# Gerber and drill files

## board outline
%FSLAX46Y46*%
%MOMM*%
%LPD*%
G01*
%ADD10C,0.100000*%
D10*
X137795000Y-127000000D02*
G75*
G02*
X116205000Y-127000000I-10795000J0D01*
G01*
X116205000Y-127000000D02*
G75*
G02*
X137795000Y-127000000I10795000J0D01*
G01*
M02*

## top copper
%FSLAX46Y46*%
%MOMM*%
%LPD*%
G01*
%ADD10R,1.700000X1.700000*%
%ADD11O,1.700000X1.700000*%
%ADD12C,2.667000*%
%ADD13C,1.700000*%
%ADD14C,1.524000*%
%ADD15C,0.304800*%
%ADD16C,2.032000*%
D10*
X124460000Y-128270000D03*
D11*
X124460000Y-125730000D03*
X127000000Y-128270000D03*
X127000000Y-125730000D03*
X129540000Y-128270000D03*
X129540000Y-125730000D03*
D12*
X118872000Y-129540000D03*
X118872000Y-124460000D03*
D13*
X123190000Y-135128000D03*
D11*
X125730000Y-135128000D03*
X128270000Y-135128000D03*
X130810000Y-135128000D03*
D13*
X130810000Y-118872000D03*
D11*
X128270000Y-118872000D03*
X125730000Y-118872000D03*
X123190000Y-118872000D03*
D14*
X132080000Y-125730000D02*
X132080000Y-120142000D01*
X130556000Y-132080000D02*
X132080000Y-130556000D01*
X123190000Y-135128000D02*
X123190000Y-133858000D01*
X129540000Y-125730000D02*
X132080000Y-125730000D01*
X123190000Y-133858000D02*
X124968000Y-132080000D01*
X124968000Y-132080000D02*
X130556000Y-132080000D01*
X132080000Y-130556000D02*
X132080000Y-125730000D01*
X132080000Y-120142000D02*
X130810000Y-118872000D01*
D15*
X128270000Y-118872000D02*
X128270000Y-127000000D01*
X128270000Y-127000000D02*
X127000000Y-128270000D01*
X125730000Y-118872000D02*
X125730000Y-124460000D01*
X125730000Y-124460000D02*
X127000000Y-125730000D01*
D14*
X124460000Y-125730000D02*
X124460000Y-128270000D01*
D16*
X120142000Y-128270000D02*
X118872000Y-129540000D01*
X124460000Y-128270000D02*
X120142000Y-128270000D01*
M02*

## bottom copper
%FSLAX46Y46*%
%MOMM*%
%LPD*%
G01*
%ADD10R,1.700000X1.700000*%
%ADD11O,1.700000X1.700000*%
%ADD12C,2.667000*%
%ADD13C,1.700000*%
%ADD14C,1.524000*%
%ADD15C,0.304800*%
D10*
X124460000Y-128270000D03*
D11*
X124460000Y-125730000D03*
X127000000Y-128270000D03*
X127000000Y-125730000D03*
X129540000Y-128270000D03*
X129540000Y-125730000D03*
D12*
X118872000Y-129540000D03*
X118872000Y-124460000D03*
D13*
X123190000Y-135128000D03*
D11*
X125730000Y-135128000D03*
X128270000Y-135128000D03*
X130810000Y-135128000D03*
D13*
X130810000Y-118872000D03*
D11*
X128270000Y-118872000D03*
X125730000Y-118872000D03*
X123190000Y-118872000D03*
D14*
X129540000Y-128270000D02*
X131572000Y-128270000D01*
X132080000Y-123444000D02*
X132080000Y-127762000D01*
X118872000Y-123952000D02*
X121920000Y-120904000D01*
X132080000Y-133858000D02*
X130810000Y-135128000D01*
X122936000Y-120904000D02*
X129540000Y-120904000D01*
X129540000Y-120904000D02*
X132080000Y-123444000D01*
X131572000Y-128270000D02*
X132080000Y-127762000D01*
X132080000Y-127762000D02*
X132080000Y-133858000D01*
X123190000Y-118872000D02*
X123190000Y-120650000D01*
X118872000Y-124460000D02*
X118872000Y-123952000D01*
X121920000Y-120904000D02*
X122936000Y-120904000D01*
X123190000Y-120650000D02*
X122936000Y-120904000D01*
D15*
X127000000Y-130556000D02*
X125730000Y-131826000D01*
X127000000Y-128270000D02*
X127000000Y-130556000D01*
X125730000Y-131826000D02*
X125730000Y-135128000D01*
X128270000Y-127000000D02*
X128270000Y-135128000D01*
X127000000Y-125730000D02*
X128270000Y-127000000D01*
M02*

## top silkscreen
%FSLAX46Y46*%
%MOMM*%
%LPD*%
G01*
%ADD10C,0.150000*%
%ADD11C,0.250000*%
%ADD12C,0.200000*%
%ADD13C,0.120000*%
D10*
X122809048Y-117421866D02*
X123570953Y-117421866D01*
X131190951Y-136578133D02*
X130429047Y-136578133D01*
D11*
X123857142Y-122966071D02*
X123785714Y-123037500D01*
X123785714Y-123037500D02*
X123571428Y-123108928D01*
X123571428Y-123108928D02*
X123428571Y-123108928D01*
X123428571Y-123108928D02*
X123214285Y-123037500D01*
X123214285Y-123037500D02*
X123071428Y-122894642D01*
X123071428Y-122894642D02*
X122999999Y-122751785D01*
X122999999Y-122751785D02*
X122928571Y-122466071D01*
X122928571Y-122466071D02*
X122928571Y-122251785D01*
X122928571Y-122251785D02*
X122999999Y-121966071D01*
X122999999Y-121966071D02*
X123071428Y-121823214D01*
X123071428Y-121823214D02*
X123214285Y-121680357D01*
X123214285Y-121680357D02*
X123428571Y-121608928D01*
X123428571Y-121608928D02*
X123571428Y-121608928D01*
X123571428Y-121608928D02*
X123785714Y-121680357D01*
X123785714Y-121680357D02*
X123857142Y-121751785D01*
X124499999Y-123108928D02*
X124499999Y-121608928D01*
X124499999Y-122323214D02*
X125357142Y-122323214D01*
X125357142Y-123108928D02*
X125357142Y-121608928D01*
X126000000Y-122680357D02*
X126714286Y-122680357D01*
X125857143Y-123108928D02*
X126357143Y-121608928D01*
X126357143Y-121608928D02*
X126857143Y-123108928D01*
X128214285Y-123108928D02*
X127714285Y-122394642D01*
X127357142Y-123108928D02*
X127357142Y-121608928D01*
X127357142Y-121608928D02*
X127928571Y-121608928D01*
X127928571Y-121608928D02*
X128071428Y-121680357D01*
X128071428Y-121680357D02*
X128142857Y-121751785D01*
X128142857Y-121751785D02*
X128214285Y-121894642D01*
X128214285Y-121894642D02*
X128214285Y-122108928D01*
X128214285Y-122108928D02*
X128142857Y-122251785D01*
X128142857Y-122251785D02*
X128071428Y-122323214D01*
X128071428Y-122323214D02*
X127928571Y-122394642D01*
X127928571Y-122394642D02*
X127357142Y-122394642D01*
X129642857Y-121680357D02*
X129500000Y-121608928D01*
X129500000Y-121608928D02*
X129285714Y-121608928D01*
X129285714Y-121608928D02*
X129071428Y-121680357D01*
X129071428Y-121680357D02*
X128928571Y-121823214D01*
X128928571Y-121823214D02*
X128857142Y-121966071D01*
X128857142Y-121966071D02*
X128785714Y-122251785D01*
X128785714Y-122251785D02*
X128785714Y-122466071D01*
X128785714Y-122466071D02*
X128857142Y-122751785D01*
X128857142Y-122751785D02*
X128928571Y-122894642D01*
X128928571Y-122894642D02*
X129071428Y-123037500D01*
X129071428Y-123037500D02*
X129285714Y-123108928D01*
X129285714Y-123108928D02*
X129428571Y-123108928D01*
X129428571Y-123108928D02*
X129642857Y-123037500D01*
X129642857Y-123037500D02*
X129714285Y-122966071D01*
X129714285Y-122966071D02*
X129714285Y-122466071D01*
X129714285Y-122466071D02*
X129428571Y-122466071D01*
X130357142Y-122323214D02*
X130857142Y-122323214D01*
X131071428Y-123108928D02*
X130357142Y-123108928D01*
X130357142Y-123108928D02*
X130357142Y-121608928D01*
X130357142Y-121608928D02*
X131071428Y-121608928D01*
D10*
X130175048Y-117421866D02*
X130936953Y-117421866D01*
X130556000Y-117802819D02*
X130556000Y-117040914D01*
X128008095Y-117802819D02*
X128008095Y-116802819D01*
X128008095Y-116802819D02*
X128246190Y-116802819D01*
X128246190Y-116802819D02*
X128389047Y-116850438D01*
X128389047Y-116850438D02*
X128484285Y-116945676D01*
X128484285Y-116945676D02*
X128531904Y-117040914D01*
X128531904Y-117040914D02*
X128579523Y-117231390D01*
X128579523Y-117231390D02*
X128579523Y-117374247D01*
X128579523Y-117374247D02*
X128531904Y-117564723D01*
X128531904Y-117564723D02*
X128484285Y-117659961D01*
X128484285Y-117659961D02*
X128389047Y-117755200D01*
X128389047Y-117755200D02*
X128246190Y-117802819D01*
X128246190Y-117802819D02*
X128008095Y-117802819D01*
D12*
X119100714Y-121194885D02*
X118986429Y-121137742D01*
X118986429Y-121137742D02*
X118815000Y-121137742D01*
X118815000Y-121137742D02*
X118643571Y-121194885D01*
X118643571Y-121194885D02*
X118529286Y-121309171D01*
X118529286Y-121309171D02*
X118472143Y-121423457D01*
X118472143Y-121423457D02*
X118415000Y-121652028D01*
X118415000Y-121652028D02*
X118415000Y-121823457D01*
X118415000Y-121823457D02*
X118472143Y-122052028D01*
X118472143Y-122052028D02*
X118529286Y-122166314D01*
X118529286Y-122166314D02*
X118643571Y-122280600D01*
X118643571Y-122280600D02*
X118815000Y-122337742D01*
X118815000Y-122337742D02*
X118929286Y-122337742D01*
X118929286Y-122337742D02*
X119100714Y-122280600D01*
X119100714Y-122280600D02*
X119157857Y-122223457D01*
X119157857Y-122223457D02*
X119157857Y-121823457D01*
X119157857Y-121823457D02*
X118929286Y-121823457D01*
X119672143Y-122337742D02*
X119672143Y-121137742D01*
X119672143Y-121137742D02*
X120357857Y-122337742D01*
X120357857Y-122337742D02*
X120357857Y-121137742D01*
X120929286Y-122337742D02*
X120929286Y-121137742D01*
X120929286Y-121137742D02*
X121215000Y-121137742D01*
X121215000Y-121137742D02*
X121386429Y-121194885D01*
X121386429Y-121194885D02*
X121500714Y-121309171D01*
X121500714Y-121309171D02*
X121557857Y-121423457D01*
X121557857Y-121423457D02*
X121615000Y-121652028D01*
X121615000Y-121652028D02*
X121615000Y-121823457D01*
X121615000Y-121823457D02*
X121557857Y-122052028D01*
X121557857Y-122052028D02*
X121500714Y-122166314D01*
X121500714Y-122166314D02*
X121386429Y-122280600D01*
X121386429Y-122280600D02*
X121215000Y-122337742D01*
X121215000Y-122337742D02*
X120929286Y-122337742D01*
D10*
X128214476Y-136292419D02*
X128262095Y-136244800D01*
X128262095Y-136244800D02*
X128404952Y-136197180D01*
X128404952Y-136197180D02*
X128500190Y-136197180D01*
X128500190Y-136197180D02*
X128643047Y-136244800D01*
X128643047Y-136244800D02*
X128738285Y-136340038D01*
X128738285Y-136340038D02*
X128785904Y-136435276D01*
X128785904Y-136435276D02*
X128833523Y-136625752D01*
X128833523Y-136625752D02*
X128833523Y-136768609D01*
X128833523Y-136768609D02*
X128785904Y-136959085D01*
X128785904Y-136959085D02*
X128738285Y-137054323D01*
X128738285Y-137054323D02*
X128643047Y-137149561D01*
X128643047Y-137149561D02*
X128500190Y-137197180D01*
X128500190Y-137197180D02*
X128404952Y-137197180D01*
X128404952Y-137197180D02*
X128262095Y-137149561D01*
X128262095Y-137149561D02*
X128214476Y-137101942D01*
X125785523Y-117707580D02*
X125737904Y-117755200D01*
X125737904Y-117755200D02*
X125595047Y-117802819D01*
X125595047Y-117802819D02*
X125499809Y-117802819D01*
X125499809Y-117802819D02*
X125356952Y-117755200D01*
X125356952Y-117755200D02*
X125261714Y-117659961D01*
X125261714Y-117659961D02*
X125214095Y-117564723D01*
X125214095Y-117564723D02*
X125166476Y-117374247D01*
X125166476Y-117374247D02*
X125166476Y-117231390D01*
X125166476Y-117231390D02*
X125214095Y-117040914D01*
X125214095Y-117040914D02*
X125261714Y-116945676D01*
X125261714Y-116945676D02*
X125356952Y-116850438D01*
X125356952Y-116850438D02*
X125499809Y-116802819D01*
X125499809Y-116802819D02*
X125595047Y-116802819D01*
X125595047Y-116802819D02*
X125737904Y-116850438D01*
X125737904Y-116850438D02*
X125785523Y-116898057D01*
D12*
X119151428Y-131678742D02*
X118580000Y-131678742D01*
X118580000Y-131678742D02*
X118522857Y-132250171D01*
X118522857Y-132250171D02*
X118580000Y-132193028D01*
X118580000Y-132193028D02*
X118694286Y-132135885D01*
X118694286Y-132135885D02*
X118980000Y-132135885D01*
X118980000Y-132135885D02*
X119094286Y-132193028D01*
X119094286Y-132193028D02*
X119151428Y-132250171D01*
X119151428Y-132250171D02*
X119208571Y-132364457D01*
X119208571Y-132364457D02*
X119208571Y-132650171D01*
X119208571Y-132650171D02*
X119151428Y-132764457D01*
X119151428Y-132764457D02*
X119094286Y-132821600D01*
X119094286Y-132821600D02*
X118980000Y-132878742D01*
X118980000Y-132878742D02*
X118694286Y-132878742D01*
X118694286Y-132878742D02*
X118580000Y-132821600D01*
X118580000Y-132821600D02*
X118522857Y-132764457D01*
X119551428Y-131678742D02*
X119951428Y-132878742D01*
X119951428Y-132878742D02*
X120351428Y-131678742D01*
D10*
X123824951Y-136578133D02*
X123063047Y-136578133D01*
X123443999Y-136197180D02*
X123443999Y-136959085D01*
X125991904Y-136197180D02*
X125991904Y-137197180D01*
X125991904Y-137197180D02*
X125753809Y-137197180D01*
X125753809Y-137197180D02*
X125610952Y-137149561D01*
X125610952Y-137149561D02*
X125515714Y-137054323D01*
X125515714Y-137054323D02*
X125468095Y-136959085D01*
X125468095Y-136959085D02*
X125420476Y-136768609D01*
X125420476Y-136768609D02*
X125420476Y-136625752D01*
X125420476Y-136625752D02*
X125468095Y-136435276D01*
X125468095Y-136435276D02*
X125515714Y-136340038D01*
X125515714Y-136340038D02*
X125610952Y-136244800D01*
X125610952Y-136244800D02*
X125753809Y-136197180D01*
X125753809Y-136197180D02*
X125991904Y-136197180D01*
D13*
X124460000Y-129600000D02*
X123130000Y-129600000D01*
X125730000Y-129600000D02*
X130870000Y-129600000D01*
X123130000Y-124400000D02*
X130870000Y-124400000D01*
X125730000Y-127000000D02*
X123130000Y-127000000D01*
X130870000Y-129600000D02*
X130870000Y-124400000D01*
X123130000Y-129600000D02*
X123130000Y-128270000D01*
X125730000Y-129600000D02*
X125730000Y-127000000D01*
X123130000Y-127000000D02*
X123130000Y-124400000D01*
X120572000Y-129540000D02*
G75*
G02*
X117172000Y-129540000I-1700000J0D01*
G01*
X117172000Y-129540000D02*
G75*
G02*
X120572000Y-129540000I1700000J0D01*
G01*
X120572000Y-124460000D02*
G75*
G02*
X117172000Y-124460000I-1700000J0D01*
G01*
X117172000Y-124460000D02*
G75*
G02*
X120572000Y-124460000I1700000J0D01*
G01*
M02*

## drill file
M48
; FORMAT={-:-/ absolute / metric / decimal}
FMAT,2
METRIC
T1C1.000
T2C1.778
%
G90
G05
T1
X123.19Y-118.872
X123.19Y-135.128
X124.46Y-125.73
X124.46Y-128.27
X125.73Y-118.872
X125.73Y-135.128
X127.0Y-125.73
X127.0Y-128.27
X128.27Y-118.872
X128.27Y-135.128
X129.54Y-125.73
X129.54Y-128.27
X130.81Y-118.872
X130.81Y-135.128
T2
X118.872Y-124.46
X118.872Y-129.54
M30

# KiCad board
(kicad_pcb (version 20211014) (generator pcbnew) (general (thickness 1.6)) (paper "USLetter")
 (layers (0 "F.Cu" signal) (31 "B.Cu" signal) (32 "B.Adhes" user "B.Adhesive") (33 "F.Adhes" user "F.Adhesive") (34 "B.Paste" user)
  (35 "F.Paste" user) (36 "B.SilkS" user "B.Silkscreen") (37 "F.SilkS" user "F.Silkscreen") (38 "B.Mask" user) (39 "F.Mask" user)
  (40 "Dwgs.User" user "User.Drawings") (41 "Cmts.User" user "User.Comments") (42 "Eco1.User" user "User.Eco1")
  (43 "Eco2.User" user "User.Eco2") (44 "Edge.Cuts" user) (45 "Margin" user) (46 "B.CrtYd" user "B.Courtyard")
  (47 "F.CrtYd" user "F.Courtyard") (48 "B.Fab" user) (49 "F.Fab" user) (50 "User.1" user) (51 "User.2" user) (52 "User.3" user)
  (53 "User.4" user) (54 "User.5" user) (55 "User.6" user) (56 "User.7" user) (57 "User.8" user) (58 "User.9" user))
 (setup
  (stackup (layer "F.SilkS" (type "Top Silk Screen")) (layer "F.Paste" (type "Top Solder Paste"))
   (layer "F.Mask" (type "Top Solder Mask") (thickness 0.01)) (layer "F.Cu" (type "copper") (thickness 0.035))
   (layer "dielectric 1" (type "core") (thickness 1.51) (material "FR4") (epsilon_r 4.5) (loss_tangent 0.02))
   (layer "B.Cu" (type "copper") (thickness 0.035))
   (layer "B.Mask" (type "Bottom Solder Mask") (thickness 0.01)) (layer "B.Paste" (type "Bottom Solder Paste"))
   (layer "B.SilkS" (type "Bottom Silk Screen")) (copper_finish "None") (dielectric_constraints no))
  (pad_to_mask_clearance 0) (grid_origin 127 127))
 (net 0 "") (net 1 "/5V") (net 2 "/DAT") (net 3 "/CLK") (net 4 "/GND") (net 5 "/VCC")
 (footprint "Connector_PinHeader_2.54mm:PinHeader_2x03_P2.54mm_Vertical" (layer "F.Cu") (at 124.46 128.27 90)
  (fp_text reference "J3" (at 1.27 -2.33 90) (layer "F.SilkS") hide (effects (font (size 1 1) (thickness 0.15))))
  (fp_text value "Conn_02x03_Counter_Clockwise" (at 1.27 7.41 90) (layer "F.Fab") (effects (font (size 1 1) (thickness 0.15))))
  (fp_line (start -1.33 0) (end -1.33 -1.33) (layer "F.SilkS") (width 0.12))
  (fp_line (start -1.33 1.27) (end -1.33 6.41) (layer "F.SilkS") (width 0.12))
  (fp_line (start 3.87 -1.33) (end 3.87 6.41) (layer "F.SilkS") (width 0.12))
  (fp_line (start 1.27 1.27) (end 1.27 -1.33) (layer "F.SilkS") (width 0.12))
  (fp_line (start -1.33 6.41) (end 3.87 6.41) (layer "F.SilkS") (width 0.12))
  (fp_line (start -1.33 -1.33) (end 0 -1.33) (layer "F.SilkS") (width 0.12))
  (fp_line (start -1.33 1.27) (end 1.27 1.27) (layer "F.SilkS") (width 0.12))
  (fp_line (start 1.27 -1.33) (end 3.87 -1.33) (layer "F.SilkS") (width 0.12))
  (pad "1" thru_hole rect (at 0 0 90) (size 1.7 1.7) (drill 1) (layers *.Cu *.Mask) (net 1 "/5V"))
  (pad "2" thru_hole oval (at 2.54 0 90) (size 1.7 1.7) (drill 1) (layers *.Cu *.Mask) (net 1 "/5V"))
  (pad "3" thru_hole oval (at 0 2.54 90) (size 1.7 1.7) (drill 1) (layers *.Cu *.Mask) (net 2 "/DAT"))
  (pad "4" thru_hole oval (at 2.54 2.54 90) (size 1.7 1.7) (drill 1) (layers *.Cu *.Mask) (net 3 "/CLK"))
  (pad "5" thru_hole oval (at 0 5.08 90) (size 1.7 1.7) (drill 1) (layers *.Cu *.Mask) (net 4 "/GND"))
  (pad "6" thru_hole oval (at 2.54 5.08 90) (size 1.7 1.7) (drill 1) (layers *.Cu *.Mask) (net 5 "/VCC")))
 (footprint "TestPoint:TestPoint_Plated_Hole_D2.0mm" (layer "F.Cu") (at 118.872 129.54)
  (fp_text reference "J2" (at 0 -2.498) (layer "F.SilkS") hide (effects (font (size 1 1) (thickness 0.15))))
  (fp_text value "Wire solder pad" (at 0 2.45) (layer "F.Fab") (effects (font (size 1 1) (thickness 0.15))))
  (fp_circle (center 0 0) (end 0 -1.7) (layer "F.SilkS") (width 0.12) (fill none))
  (pad "1" thru_hole circle (at 0 0) (size 2.667 2.667) (drill 1.778) (layers *.Cu *.Mask) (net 1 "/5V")))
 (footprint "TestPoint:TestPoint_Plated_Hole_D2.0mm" (layer "F.Cu") (at 118.872 124.46)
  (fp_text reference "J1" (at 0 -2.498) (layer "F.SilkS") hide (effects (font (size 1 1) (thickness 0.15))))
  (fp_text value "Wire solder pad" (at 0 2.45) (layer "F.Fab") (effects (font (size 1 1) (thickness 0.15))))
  (fp_circle (center 0 0) (end 0 -1.7) (layer "F.SilkS") (width 0.12) (fill none))
  (pad "1" thru_hole circle (at 0 0) (size 2.667 2.667) (drill 1.778) (layers *.Cu *.Mask) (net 4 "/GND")))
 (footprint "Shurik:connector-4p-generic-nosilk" (layer "F.Cu") (at 123.19 135.128 90)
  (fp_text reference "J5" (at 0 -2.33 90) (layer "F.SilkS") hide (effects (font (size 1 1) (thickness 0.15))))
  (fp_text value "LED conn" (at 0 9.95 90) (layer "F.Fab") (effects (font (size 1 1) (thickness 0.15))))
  (pad "1" thru_hole circle (at 0 0 90) (size 1.7 1.7) (drill 1) (layers *.Cu *.Mask) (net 5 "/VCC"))
  (pad "2" thru_hole oval (at 0 2.54 90) (size 1.7 1.7) (drill 1) (layers *.Cu *.Mask) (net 2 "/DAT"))
  (pad "3" thru_hole oval (at 0 5.08 90) (size 1.7 1.7) (drill 1) (layers *.Cu *.Mask) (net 3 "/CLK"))
  (pad "4" thru_hole oval (at 0 7.62 90) (size 1.7 1.7) (drill 1) (layers *.Cu *.Mask) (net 4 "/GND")))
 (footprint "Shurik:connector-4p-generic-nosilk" (layer "F.Cu") (at 130.81 118.872 -90)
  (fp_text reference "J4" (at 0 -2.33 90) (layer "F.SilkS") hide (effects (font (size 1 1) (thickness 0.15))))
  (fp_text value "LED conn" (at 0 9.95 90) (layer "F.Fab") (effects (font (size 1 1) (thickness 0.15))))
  (pad "1" thru_hole circle (at 0 0 270) (size 1.7 1.7) (drill 1) (layers *.Cu *.Mask) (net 5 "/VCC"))
  (pad "2" thru_hole oval (at 0 2.54 270) (size 1.7 1.7) (drill 1) (layers *.Cu *.Mask) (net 2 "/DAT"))
  (pad "3" thru_hole oval (at 0 5.08 270) (size 1.7 1.7) (drill 1) (layers *.Cu *.Mask) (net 3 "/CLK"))
  (pad "4" thru_hole oval (at 0 7.62 270) (size 1.7 1.7) (drill 1) (layers *.Cu *.Mask) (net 4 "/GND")))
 (gr_arc (start 137.795 127) (mid 127 137.795) (end 116.205 127) (layer "Edge.Cuts") (width 0.1))
 (gr_arc (start 116.205 127) (mid 127 116.205) (end 137.795 127) (layer "Edge.Cuts") (width 0.1))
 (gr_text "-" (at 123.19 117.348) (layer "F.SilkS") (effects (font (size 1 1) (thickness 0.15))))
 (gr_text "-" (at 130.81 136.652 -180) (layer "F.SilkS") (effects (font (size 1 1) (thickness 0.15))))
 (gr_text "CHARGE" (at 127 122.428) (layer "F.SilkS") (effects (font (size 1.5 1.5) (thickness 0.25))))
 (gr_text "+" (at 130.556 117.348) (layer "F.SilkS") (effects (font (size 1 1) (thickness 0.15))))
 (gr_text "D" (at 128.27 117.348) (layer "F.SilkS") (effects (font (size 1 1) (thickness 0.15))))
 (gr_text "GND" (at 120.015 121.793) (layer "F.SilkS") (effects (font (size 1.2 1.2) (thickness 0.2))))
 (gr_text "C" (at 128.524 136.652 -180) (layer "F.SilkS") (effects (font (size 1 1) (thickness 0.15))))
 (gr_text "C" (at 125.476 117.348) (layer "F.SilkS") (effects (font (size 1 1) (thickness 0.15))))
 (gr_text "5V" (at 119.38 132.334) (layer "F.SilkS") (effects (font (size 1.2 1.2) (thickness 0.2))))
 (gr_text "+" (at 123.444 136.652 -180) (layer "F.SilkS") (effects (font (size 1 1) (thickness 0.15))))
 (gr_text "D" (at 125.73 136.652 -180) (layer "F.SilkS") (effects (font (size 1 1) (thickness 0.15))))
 (segment (start 129.54 128.27) (end 131.572 128.27) (width 1.524) (layer "B.Cu") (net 4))
 (segment (start 132.08 123.444) (end 132.08 127.762) (width 1.524) (layer "B.Cu") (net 4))
 (segment (start 118.872 123.952) (end 121.92 120.904) (width 1.524) (layer "B.Cu") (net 4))
 (segment (start 132.08 133.858) (end 130.81 135.128) (width 1.524) (layer "B.Cu") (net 4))
 (segment (start 122.936 120.904) (end 129.54 120.904) (width 1.524) (layer "B.Cu") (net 4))
 (segment (start 129.54 120.904) (end 132.08 123.444) (width 1.524) (layer "B.Cu") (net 4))
 (segment (start 131.572 128.27) (end 132.08 127.762) (width 1.524) (layer "B.Cu") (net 4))
 (segment (start 132.08 127.762) (end 132.08 133.858) (width 1.524) (layer "B.Cu") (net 4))
 (segment (start 123.19 118.872) (end 123.19 120.65) (width 1.524) (layer "B.Cu") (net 4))
 (segment (start 118.872 124.46) (end 118.872 123.952) (width 1.524) (layer "B.Cu") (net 4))
 (segment (start 121.92 120.904) (end 122.936 120.904) (width 1.524) (layer "B.Cu") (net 4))
 (segment (start 123.19 120.65) (end 122.936 120.904) (width 1.524) (layer "B.Cu") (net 4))
 (segment (start 132.08 125.73) (end 132.08 120.142) (width 1.524) (layer "F.Cu") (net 5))
 (segment (start 130.556 132.08) (end 132.08 130.556) (width 1.524) (layer "F.Cu") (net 5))
 (segment (start 123.19 135.128) (end 123.19 133.858) (width 1.524) (layer "F.Cu") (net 5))
 (segment (start 129.54 125.73) (end 132.08 125.73) (width 1.524) (layer "F.Cu") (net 5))
 (segment (start 123.19 133.858) (end 124.968 132.08) (width 1.524) (layer "F.Cu") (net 5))
 (segment (start 124.968 132.08) (end 130.556 132.08) (width 1.524) (layer "F.Cu") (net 5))
 (segment (start 132.08 130.556) (end 132.08 125.73) (width 1.524) (layer "F.Cu") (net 5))
 (segment (start 132.08 120.142) (end 130.81 118.872) (width 1.524) (layer "F.Cu") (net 5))
 (segment (start 128.27 118.872) (end 128.27 127) (width 0.3048) (layer "F.Cu") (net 2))
 (segment (start 128.27 127) (end 127 128.27) (width 0.3048) (layer "F.Cu") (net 2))
 (segment (start 127 130.556) (end 125.73 131.826) (width 0.3048) (layer "B.Cu") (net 2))
 (segment (start 127 128.27) (end 127 130.556) (width 0.3048) (layer "B.Cu") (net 2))
 (segment (start 125.73 131.826) (end 125.73 135.128) (width 0.3048) (layer "B.Cu") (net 2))
 (segment (start 125.73 118.872) (end 125.73 124.46) (width 0.3048) (layer "F.Cu") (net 3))
 (segment (start 125.73 124.46) (end 127 125.73) (width 0.3048) (layer "F.Cu") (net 3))
 (segment (start 128.27 127) (end 128.27 135.128) (width 0.3048) (layer "B.Cu") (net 3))
 (segment (start 127 125.73) (end 128.27 127) (width 0.3048) (layer "B.Cu") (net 3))
 (segment (start 124.46 125.73) (end 124.46 128.27) (width 1.524) (layer "F.Cu") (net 1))
 (segment (start 120.142 128.27) (end 118.872 129.54) (width 2.032) (layer "F.Cu") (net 1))
 (segment (start 124.46 128.27) (end 120.142 128.27) (width 2.032) (layer "F.Cu") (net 1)))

